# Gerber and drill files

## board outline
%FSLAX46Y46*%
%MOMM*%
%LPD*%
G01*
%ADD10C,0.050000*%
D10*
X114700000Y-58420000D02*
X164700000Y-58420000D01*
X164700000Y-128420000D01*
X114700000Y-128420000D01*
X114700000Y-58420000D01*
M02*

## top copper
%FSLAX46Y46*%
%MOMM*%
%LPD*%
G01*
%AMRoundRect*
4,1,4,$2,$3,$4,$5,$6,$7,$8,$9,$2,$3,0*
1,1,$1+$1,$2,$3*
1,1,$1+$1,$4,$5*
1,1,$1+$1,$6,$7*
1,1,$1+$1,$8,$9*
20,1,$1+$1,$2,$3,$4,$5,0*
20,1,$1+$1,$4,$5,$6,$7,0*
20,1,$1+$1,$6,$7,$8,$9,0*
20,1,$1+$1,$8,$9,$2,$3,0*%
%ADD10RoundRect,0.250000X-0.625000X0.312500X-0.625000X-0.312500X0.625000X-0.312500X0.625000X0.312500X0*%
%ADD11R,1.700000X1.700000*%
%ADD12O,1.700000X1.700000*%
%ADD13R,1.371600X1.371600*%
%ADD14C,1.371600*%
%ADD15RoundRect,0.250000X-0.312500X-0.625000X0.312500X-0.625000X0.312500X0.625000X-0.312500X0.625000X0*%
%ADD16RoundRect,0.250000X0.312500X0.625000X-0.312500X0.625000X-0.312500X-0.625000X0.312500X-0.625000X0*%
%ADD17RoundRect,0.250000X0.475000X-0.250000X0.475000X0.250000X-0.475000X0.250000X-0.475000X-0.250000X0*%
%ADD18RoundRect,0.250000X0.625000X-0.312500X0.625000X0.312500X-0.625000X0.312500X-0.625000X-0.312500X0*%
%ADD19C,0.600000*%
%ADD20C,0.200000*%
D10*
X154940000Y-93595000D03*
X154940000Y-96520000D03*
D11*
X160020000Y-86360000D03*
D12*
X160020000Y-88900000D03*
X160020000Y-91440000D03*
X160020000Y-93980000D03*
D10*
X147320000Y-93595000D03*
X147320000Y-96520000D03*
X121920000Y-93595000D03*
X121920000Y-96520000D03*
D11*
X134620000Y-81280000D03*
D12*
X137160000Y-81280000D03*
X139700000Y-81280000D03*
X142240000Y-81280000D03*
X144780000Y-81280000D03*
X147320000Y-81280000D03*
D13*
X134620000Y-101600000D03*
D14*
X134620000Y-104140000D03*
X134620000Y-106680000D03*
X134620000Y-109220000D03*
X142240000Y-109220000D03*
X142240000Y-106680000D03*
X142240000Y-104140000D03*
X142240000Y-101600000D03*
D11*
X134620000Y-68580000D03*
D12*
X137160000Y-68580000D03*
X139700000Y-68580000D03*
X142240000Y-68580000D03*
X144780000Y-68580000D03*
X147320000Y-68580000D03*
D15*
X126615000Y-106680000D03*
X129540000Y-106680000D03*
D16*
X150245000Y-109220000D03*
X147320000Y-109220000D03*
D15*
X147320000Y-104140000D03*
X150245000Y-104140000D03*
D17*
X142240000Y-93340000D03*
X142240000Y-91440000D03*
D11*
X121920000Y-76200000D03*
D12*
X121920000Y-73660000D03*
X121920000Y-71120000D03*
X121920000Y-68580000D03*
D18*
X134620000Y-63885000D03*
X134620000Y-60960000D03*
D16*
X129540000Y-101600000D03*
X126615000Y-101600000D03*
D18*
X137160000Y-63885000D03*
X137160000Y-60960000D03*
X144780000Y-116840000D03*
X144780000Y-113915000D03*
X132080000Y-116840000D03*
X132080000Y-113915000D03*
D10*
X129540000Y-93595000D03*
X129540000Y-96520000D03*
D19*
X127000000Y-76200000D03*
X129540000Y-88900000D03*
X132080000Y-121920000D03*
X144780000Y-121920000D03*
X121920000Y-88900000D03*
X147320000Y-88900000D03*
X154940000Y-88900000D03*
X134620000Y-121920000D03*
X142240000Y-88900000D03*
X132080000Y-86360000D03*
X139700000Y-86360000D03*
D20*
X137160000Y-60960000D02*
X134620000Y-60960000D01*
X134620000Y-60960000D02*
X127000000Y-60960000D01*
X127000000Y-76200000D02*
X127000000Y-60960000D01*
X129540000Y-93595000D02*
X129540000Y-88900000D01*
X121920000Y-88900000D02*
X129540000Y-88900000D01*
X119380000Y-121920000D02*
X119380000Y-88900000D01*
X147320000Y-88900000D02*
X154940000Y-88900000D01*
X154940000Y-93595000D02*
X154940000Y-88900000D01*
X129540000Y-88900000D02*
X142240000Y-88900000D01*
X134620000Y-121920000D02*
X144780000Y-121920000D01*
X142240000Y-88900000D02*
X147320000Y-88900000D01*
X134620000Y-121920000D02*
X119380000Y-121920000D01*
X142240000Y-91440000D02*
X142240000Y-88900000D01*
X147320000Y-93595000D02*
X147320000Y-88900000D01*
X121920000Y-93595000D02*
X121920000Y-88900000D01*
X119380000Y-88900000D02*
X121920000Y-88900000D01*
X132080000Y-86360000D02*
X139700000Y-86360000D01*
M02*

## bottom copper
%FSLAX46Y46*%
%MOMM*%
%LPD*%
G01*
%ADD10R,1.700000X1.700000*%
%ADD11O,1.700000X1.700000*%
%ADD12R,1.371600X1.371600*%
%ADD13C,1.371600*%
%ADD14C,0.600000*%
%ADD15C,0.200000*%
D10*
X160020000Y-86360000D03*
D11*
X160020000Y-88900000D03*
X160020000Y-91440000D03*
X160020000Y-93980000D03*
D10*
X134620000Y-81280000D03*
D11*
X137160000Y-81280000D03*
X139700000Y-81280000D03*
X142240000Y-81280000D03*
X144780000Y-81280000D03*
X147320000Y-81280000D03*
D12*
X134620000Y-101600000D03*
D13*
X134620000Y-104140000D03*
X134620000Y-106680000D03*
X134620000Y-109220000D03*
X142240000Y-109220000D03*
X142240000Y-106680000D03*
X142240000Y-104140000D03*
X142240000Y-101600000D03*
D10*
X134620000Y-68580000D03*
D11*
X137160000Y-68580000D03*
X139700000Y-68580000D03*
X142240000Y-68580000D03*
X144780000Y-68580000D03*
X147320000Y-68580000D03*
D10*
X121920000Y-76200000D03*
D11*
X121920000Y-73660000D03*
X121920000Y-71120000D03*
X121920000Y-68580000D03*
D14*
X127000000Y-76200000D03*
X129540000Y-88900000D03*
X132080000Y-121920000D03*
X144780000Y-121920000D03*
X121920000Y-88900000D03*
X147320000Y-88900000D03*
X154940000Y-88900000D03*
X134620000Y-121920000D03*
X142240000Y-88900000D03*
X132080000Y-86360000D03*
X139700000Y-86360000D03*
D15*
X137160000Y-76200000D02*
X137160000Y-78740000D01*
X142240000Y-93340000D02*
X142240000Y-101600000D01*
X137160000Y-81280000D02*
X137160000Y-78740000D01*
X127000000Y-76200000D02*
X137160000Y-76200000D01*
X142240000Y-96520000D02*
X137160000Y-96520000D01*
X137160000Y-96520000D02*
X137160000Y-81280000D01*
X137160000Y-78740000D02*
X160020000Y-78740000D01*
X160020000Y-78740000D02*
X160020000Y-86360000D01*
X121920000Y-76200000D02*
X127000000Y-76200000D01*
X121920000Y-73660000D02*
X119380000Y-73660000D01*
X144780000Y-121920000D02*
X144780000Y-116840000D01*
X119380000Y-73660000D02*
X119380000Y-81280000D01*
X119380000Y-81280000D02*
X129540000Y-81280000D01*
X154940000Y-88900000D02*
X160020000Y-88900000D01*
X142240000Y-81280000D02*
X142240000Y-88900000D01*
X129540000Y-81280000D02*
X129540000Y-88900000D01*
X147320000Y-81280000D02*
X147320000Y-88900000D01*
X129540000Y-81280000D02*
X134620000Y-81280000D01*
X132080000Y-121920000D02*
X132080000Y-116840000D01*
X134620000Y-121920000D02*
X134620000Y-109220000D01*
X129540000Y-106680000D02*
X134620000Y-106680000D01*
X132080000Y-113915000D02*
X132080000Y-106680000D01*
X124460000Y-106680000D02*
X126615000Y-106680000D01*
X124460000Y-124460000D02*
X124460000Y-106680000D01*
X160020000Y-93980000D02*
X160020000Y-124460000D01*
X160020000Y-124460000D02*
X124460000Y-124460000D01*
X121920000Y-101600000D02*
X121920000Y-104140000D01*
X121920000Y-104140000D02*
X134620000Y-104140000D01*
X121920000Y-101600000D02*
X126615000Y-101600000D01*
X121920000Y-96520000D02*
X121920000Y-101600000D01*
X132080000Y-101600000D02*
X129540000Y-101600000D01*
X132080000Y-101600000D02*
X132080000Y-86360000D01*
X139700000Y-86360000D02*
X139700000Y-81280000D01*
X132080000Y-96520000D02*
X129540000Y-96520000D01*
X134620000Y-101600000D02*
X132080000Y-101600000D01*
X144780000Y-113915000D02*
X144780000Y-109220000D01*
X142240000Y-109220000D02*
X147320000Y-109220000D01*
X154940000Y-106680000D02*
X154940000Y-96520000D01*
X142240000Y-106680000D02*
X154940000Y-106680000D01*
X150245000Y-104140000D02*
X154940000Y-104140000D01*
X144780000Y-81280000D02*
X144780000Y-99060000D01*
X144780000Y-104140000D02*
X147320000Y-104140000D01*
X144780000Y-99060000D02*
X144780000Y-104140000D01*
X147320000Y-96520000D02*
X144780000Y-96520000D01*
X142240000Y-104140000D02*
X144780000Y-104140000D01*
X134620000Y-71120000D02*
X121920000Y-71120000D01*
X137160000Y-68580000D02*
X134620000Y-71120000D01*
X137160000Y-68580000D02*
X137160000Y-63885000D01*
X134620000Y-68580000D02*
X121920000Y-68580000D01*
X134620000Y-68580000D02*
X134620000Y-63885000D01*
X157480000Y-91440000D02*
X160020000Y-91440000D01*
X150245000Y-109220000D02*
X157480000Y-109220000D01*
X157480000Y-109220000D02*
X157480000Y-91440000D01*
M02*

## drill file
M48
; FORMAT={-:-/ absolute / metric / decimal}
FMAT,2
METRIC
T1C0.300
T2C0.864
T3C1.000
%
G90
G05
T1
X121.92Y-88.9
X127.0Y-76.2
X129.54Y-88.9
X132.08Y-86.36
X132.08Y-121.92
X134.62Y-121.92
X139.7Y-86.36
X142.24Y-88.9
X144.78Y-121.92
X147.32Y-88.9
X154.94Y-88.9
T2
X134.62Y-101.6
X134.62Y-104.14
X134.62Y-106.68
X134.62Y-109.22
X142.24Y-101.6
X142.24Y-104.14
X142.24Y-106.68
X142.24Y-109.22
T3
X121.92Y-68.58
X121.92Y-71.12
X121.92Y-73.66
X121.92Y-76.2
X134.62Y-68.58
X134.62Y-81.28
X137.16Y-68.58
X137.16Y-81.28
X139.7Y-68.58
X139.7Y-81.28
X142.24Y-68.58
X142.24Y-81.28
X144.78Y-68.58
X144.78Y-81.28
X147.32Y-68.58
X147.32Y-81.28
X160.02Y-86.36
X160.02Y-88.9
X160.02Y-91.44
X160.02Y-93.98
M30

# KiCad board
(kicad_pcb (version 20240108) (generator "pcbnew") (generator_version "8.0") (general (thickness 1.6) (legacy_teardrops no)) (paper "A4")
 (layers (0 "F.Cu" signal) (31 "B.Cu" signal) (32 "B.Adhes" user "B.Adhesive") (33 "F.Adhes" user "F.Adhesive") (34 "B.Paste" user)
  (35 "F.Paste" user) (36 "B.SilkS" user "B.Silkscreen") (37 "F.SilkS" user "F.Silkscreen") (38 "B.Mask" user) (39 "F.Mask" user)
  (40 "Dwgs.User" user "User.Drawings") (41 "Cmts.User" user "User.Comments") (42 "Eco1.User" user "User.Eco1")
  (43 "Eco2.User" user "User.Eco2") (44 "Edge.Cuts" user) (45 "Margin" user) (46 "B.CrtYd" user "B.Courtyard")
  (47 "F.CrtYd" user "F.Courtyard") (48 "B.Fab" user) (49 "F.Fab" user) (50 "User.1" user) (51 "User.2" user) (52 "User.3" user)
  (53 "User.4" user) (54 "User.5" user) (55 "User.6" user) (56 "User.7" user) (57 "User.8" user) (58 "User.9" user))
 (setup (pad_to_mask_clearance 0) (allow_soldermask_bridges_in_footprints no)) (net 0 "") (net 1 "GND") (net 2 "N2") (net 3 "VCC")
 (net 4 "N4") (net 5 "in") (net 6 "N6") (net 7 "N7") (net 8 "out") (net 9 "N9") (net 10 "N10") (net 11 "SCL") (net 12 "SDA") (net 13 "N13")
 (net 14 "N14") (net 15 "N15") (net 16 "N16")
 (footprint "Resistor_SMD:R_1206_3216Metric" (layer "F.Cu") (at 154.94 95.0575 -90)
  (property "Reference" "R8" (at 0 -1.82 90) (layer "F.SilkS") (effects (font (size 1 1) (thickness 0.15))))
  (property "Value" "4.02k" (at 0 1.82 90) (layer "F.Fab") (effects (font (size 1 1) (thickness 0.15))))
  (pad "1" smd roundrect (at -1.4625 0 270) (size 1.125 1.75) (layers "F.Cu" "F.Paste" "F.Mask") (roundrect_rratio 0.222222) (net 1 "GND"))
  (pad "2" smd roundrect (at 1.4625 0 270) (size 1.125 1.75) (layers "F.Cu" "F.Paste" "F.Mask") (roundrect_rratio 0.222222) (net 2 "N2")))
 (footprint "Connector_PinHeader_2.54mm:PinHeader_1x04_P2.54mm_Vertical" (layer "F.Cu") (at 160.02 86.36)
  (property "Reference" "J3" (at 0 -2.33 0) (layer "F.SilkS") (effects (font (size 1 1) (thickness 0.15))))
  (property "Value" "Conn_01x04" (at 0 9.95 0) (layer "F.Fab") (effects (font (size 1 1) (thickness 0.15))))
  (pad "1" thru_hole rect (at 0 0) (size 1.7 1.7) (drill 1) (layers "*.Cu" "*.Mask") (remove_unused_layers no) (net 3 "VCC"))
  (pad "2" thru_hole oval (at 0 2.54) (size 1.7 1.7) (drill 1) (layers "*.Cu" "*.Mask") (remove_unused_layers no) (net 1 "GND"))
  (pad "3" thru_hole oval (at 0 5.08) (size 1.7 1.7) (drill 1) (layers "*.Cu" "*.Mask") (remove_unused_layers no) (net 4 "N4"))
  (pad "4" thru_hole oval (at 0 7.62) (size 1.7 1.7) (drill 1) (layers "*.Cu" "*.Mask") (remove_unused_layers no) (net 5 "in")))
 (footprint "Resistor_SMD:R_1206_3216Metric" (layer "F.Cu") (at 147.32 95.0575 -90)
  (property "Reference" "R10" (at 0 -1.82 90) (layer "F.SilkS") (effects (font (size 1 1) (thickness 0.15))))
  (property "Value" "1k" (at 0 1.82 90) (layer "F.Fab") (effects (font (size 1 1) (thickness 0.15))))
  (pad "1" smd roundrect (at -1.4625 0 270) (size 1.125 1.75) (layers "F.Cu" "F.Paste" "F.Mask") (roundrect_rratio 0.222222) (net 1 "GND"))
  (pad "2" smd roundrect (at 1.4625 0 270) (size 1.125 1.75) (layers "F.Cu" "F.Paste" "F.Mask") (roundrect_rratio 0.222222) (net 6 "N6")))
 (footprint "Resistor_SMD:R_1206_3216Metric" (layer "F.Cu") (at 121.92 95.0575 -90)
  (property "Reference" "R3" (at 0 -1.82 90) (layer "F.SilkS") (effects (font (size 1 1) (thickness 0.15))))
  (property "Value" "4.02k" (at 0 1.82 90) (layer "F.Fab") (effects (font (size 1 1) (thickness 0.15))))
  (pad "1" smd roundrect (at -1.4625 0 270) (size 1.125 1.75) (layers "F.Cu" "F.Paste" "F.Mask") (roundrect_rratio 0.222222) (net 1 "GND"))
  (pad "2" smd roundrect (at 1.4625 0 270) (size 1.125 1.75) (layers "F.Cu" "F.Paste" "F.Mask") (roundrect_rratio 0.222222) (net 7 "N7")))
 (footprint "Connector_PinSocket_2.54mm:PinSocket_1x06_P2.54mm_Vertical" (layer "F.Cu") (at 134.62 81.28 90)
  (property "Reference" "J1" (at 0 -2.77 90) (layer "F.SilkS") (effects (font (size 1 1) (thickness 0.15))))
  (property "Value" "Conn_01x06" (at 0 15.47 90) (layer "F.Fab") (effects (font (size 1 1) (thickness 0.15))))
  (pad "1" thru_hole rect (at 0 0 90) (size 1.7 1.7) (drill 1) (layers "*.Cu" "*.Mask") (remove_unused_layers no) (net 1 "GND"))
  (pad "2" thru_hole oval (at 0 2.54 90) (size 1.7 1.7) (drill 1) (layers "*.Cu" "*.Mask") (remove_unused_layers no) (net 3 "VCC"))
  (pad "3" thru_hole oval (at 0 5.08 90) (size 1.7 1.7) (drill 1) (layers "*.Cu" "*.Mask") (remove_unused_layers no) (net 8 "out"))
  (pad "4" thru_hole oval (at 0 7.62 90) (size 1.7 1.7) (drill 1) (layers "*.Cu" "*.Mask") (remove_unused_layers no) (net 1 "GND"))
  (pad "5" thru_hole oval (at 0 10.16 90) (size 1.7 1.7) (drill 1) (layers "*.Cu" "*.Mask") (remove_unused_layers no) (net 6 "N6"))
  (pad "6" thru_hole oval (at 0 12.7 90) (size 1.7 1.7) (drill 1) (layers "*.Cu" "*.Mask") (remove_unused_layers no) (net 1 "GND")))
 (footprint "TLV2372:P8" (layer "F.Cu") (at 142.24 109.22)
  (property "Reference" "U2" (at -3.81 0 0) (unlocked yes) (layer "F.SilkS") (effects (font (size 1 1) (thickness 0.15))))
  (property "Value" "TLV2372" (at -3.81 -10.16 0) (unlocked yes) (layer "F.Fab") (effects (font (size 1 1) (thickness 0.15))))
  (pad "1" thru_hole rect (at -7.62 -7.62) (size 1.3716 1.3716) (drill 0.8636) (layers "*.Cu" "*.Mask") (remove_unused_layers no)
   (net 8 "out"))
  (pad "2" thru_hole circle (at -7.62 -5.08) (size 1.3716 1.3716) (drill 0.8636) (layers "*.Cu" "*.Mask") (remove_unused_layers no)
   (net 7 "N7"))
  (pad "3" thru_hole circle (at -7.62 -2.54) (size 1.3716 1.3716) (drill 0.8636) (layers "*.Cu" "*.Mask") (remove_unused_layers no)
   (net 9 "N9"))
  (pad "4" thru_hole circle (at -7.62 0) (size 1.3716 1.3716) (drill 0.8636) (layers "*.Cu" "*.Mask") (remove_unused_layers no)
   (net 1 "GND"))
  (pad "5" thru_hole circle (at 0 0) (size 1.3716 1.3716) (drill 0.8636) (layers "*.Cu" "*.Mask") (remove_unused_layers no) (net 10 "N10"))
  (pad "6" thru_hole circle (at 0 -2.54) (size 1.3716 1.3716) (drill 0.8636) (layers "*.Cu" "*.Mask") (remove_unused_layers no) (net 2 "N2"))
  (pad "7" thru_hole circle (at 0 -5.08) (size 1.3716 1.3716) (drill 0.8636) (layers "*.Cu" "*.Mask") (remove_unused_layers no) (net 6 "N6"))
  (pad "8" thru_hole circle (at 0 -7.62) (size 1.3716 1.3716) (drill 0.8636) (layers "*.Cu" "*.Mask") (remove_unused_layers no)
   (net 3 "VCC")))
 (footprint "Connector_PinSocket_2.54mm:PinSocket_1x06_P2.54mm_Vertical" (layer "F.Cu") (at 134.62 68.58 90)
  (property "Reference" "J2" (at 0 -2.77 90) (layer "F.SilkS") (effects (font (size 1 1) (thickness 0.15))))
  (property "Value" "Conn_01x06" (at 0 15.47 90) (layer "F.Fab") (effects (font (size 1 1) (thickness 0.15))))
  (pad "1" thru_hole rect (at 0 0 90) (size 1.7 1.7) (drill 1) (layers "*.Cu" "*.Mask") (remove_unused_layers no) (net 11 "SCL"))
  (pad "2" thru_hole oval (at 0 2.54 90) (size 1.7 1.7) (drill 1) (layers "*.Cu" "*.Mask") (remove_unused_layers no) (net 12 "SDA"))
  (pad "3" thru_hole oval (at 0 5.08 90) (size 1.7 1.7) (drill 1) (layers "*.Cu" "*.Mask") (remove_unused_layers no) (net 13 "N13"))
  (pad "4" thru_hole oval (at 0 7.62 90) (size 1.7 1.7) (drill 1) (layers "*.Cu" "*.Mask") (remove_unused_layers no) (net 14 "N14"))
  (pad "5" thru_hole oval (at 0 10.16 90) (size 1.7 1.7) (drill 1) (layers "*.Cu" "*.Mask") (remove_unused_layers no) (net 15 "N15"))
  (pad "6" thru_hole oval (at 0 12.7 90) (size 1.7 1.7) (drill 1) (layers "*.Cu" "*.Mask") (remove_unused_layers no) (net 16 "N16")))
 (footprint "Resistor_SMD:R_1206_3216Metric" (layer "F.Cu") (at 128.0775 106.68)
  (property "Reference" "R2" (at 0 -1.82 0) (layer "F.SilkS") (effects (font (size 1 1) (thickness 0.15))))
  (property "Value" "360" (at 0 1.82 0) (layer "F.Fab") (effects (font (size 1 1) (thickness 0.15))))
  (pad "1" smd roundrect (at -1.4625 0) (size 1.125 1.75) (layers "F.Cu" "F.Paste" "F.Mask") (roundrect_rratio 0.222222) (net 5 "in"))
  (pad "2" smd roundrect (at 1.4625 0) (size 1.125 1.75) (layers "F.Cu" "F.Paste" "F.Mask") (roundrect_rratio 0.222222) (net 9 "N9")))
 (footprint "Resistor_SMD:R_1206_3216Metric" (layer "F.Cu") (at 148.7825 109.22 180)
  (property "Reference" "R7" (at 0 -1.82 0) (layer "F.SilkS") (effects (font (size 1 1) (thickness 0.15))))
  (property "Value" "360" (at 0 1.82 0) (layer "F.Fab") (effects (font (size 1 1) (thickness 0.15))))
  (pad "1" smd roundrect (at -1.4625 0 180) (size 1.125 1.75) (layers "F.Cu" "F.Paste" "F.Mask") (roundrect_rratio 0.222222) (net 4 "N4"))
  (pad "2" smd roundrect (at 1.4625 0 180) (size 1.125 1.75) (layers "F.Cu" "F.Paste" "F.Mask") (roundrect_rratio 0.222222) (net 10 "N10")))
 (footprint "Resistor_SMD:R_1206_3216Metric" (layer "F.Cu") (at 148.7825 104.14)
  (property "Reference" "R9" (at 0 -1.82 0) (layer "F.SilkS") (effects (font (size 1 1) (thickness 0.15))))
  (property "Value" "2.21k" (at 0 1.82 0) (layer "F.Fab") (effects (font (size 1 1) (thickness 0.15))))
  (pad "1" smd roundrect (at -1.4625 0) (size 1.125 1.75) (layers "F.Cu" "F.Paste" "F.Mask") (roundrect_rratio 0.222222) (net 6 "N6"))
  (pad "2" smd roundrect (at 1.4625 0) (size 1.125 1.75) (layers "F.Cu" "F.Paste" "F.Mask") (roundrect_rratio 0.222222) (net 2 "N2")))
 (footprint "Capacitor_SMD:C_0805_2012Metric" (layer "F.Cu") (at 142.24 92.39 90)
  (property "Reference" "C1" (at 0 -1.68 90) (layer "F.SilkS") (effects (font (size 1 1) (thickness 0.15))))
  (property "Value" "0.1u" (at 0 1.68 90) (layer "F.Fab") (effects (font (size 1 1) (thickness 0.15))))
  (pad "1" smd roundrect (at -0.95 0 90) (size 1 1.45) (layers "F.Cu" "F.Paste" "F.Mask") (roundrect_rratio 0.25) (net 3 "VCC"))
  (pad "2" smd roundrect (at 0.95 0 90) (size 1 1.45) (layers "F.Cu" "F.Paste" "F.Mask") (roundrect_rratio 0.25) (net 1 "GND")))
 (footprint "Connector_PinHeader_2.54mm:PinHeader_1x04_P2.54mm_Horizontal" (layer "F.Cu") (at 121.92 76.2 180)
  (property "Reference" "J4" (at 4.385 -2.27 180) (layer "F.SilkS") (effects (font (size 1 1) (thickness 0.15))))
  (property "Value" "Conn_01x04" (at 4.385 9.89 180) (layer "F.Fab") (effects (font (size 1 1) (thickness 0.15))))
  (pad "1" thru_hole rect (at 0 0 180) (size 1.7 1.7) (drill 1) (layers "*.Cu" "*.Mask") (remove_unused_layers no) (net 3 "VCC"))
  (pad "2" thru_hole oval (at 0 2.54 180) (size 1.7 1.7) (drill 1) (layers "*.Cu" "*.Mask") (remove_unused_layers no) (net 1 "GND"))
  (pad "3" thru_hole oval (at 0 5.08 180) (size 1.7 1.7) (drill 1) (layers "*.Cu" "*.Mask") (remove_unused_layers no) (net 12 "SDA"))
  (pad "4" thru_hole oval (at 0 7.62 180) (size 1.7 1.7) (drill 1) (layers "*.Cu" "*.Mask") (remove_unused_layers no) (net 11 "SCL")))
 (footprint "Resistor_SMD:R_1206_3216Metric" (layer "F.Cu") (at 134.62 62.4225 90)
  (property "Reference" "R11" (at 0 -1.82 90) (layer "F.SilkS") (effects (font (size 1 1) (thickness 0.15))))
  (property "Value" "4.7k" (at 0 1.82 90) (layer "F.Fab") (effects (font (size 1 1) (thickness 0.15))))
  (pad "1" smd roundrect (at -1.4625 0 90) (size 1.125 1.75) (layers "F.Cu" "F.Paste" "F.Mask") (roundrect_rratio 0.222222) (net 11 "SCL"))
  (pad "2" smd roundrect (at 1.4625 0 90) (size 1.125 1.75) (layers "F.Cu" "F.Paste" "F.Mask") (roundrect_rratio 0.222222) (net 3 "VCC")))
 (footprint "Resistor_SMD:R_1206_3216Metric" (layer "F.Cu") (at 128.0775 101.6 180)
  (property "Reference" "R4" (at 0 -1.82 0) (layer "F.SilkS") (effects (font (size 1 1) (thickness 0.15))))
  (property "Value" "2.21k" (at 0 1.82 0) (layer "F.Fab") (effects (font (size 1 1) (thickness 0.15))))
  (pad "1" smd roundrect (at -1.4625 0 180) (size 1.125 1.75) (layers "F.Cu" "F.Paste" "F.Mask") (roundrect_rratio 0.222222) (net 8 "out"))
  (pad "2" smd roundrect (at 1.4625 0 180) (size 1.125 1.75) (layers "F.Cu" "F.Paste" "F.Mask") (roundrect_rratio 0.222222) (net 7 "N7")))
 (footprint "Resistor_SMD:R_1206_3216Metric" (layer "F.Cu") (at 137.16 62.4225 90)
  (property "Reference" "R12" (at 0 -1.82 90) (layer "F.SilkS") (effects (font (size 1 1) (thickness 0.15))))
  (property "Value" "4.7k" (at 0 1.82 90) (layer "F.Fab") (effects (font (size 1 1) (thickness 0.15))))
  (pad "1" smd roundrect (at -1.4625 0 90) (size 1.125 1.75) (layers "F.Cu" "F.Paste" "F.Mask") (roundrect_rratio 0.222222) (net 12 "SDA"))
  (pad "2" smd roundrect (at 1.4625 0 90) (size 1.125 1.75) (layers "F.Cu" "F.Paste" "F.Mask") (roundrect_rratio 0.222222) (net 3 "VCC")))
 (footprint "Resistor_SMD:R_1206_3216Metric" (layer "F.Cu") (at 144.78 115.3775 90)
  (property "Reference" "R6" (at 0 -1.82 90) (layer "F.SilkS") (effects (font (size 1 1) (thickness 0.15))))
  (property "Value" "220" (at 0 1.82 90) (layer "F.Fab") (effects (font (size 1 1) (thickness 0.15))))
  (pad "1" smd roundrect (at -1.4625 0 90) (size 1.125 1.75) (layers "F.Cu" "F.Paste" "F.Mask") (roundrect_rratio 0.222222) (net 1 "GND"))
  (pad "2" smd roundrect (at 1.4625 0 90) (size 1.125 1.75) (layers "F.Cu" "F.Paste" "F.Mask") (roundrect_rratio 0.222222) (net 10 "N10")))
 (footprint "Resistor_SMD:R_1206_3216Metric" (layer "F.Cu") (at 132.08 115.3775 90)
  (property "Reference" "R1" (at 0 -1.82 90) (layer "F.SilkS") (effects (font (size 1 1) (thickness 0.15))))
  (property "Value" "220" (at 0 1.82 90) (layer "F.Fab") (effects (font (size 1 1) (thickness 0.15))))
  (pad "1" smd roundrect (at -1.4625 0 90) (size 1.125 1.75) (layers "F.Cu" "F.Paste" "F.Mask") (roundrect_rratio 0.222222) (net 1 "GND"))
  (pad "2" smd roundrect (at 1.4625 0 90) (size 1.125 1.75) (layers "F.Cu" "F.Paste" "F.Mask") (roundrect_rratio 0.222222) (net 9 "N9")))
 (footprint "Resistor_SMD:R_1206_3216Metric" (layer "F.Cu") (at 129.54 95.0575 -90)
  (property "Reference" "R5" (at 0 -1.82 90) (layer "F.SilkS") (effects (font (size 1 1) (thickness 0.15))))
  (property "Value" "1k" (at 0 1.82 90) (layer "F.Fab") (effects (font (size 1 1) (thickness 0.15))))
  (pad "1" smd roundrect (at -1.4625 0 270) (size 1.125 1.75) (layers "F.Cu" "F.Paste" "F.Mask") (roundrect_rratio 0.222222) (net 1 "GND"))
  (pad "2" smd roundrect (at 1.4625 0 270) (size 1.125 1.75) (layers "F.Cu" "F.Paste" "F.Mask") (roundrect_rratio 0.222222) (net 8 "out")))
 (gr_rect (start 114.7 58.42) (end 164.7 128.42) (stroke (width 0.05) (type default)) (fill none) (layer "Edge.Cuts"))
 (segment (start 137.16 60.96) (end 134.62 60.96) (width 0.2) (layer "F.Cu") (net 3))
 (segment (start 134.62 60.96) (end 127 60.96) (width 0.2) (layer "F.Cu") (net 3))
 (segment (start 127 76.2) (end 127 60.96) (width 0.2) (layer "F.Cu") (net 3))
 (via (at 127 76.2) (size 0.6) (drill 0.3) (layers "F.Cu" "B.Cu") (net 3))
 (segment (start 137.16 76.2) (end 137.16 78.74) (width 0.2) (layer "B.Cu") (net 3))
 (segment (start 142.24 93.34) (end 142.24 101.6) (width 0.2) (layer "B.Cu") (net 3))
 (segment (start 137.16 81.28) (end 137.16 78.74) (width 0.2) (layer "B.Cu") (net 3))
 (segment (start 127 76.2) (end 137.16 76.2) (width 0.2) (layer "B.Cu") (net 3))
 (segment (start 142.24 96.52) (end 137.16 96.52) (width 0.2) (layer "B.Cu") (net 3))
 (segment (start 137.16 96.52) (end 137.16 81.28) (width 0.2) (layer "B.Cu") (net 3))
 (segment (start 137.16 78.74) (end 160.02 78.74) (width 0.2) (layer "B.Cu") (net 3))
 (segment (start 160.02 78.74) (end 160.02 86.36) (width 0.2) (layer "B.Cu") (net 3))
 (segment (start 121.92 76.2) (end 127 76.2) (width 0.2) (layer "B.Cu") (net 3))
 (segment (start 129.54 93.595) (end 129.54 88.9) (width 0.2) (layer "F.Cu") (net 1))
 (segment (start 121.92 88.9) (end 129.54 88.9) (width 0.2) (layer "F.Cu") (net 1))
 (segment (start 119.38 121.92) (end 119.38 88.9) (width 0.2) (layer "F.Cu") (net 1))
 (segment (start 147.32 88.9) (end 154.94 88.9) (width 0.2) (layer "F.Cu") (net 1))
 (segment (start 154.94 93.595) (end 154.94 88.9) (width 0.2) (layer "F.Cu") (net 1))
 (segment (start 129.54 88.9) (end 142.24 88.9) (width 0.2) (layer "F.Cu") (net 1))
 (segment (start 134.62 121.92) (end 144.78 121.92) (width 0.2) (layer "F.Cu") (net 1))
 (segment (start 142.24 88.9) (end 147.32 88.9) (width 0.2) (layer "F.Cu") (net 1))
 (segment (start 134.62 121.92) (end 119.38 121.92) (width 0.2) (layer "F.Cu") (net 1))
 (segment (start 142.24 91.44) (end 142.24 88.9) (width 0.2) (layer "F.Cu") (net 1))
 (segment (start 147.32 93.595) (end 147.32 88.9) (width 0.2) (layer "F.Cu") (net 1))
 (segment (start 121.92 93.595) (end 121.92 88.9) (width 0.2) (layer "F.Cu") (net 1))
 (segment (start 119.38 88.9) (end 121.92 88.9) (width 0.2) (layer "F.Cu") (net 1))
 (via (at 129.54 88.9) (size 0.6) (drill 0.3) (layers "F.Cu" "B.Cu") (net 1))
 (via (at 132.08 121.92) (size 0.6) (drill 0.3) (layers "F.Cu" "B.Cu") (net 1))
 (via (at 144.78 121.92) (size 0.6) (drill 0.3) (layers "F.Cu" "B.Cu") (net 1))
 (via (at 121.92 88.9) (size 0.6) (drill 0.3) (layers "F.Cu" "B.Cu") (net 1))
 (via (at 147.32 88.9) (size 0.6) (drill 0.3) (layers "F.Cu" "B.Cu") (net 1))
 (via (at 154.94 88.9) (size 0.6) (drill 0.3) (layers "F.Cu" "B.Cu") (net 1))
 (via (at 134.62 121.92) (size 0.6) (drill 0.3) (layers "F.Cu" "B.Cu") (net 1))
 (via (at 142.24 88.9) (size 0.6) (drill 0.3) (layers "F.Cu" "B.Cu") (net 1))
 (segment (start 121.92 73.66) (end 119.38 73.66) (width 0.2) (layer "B.Cu") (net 1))
 (segment (start 144.78 121.92) (end 144.78 116.84) (width 0.2) (layer "B.Cu") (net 1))
 (segment (start 119.38 73.66) (end 119.38 81.28) (width 0.2) (layer "B.Cu") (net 1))
 (segment (start 119.38 81.28) (end 129.54 81.28) (width 0.2) (layer "B.Cu") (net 1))
 (segment (start 154.94 88.9) (end 160.02 88.9) (width 0.2) (layer "B.Cu") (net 1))
 (segment (start 142.24 81.28) (end 142.24 88.9) (width 0.2) (layer "B.Cu") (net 1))
 (segment (start 129.54 81.28) (end 129.54 88.9) (width 0.2) (layer "B.Cu") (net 1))
 (segment (start 147.32 81.28) (end 147.32 88.9) (width 0.2) (layer "B.Cu") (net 1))
 (segment (start 129.54 81.28) (end 134.62 81.28) (width 0.2) (layer "B.Cu") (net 1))
 (segment (start 132.08 121.92) (end 132.08 116.84) (width 0.2) (layer "B.Cu") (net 1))
 (segment (start 134.62 121.92) (end 134.62 109.22) (width 0.2) (layer "B.Cu") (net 1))
 (segment (start 129.54 106.68) (end 134.62 106.68) (width 0.2) (layer "B.Cu") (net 9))
 (segment (start 132.08 113.915) (end 132.08 106.68) (width 0.2) (layer "B.Cu") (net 9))
 (segment (start 124.46 106.68) (end 126.615 106.68) (width 0.2) (layer "B.Cu") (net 5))
 (segment (start 124.46 124.46) (end 124.46 106.68) (width 0.2) (layer "B.Cu") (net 5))
 (segment (start 160.02 93.98) (end 160.02 124.46) (width 0.2) (layer "B.Cu") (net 5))
 (segment (start 160.02 124.46) (end 124.46 124.46) (width 0.2) (layer "B.Cu") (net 5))
 (segment (start 121.92 101.6) (end 121.92 104.14) (width 0.2) (layer "B.Cu") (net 7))
 (segment (start 121.92 104.14) (end 134.62 104.14) (width 0.2) (layer "B.Cu") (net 7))
 (segment (start 121.92 101.6) (end 126.615 101.6) (width 0.2) (layer "B.Cu") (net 7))
 (segment (start 121.92 96.52) (end 121.92 101.6) (width 0.2) (layer "B.Cu") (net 7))
 (segment (start 132.08 86.36) (end 139.7 86.36) (width 0.2) (layer "F.Cu") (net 8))
 (via (at 132.08 86.36) (size 0.6) (drill 0.3) (layers "F.Cu" "B.Cu") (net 8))
 (via (at 139.7 86.36) (size 0.6) (drill 0.3) (layers "F.Cu" "B.Cu") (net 8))
 (segment (start 132.08 101.6) (end 129.54 101.6) (width 0.2) (layer "B.Cu") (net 8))
 (segment (start 132.08 101.6) (end 132.08 86.36) (width 0.2) (layer "B.Cu") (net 8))
 (segment (start 139.7 86.36) (end 139.7 81.28) (width 0.2) (layer "B.Cu") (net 8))
 (segment (start 132.08 96.52) (end 129.54 96.52) (width 0.2) (layer "B.Cu") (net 8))
 (segment (start 134.62 101.6) (end 132.08 101.6) (width 0.2) (layer "B.Cu") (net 8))
 (segment (start 144.78 113.915) (end 144.78 109.22) (width 0.2) (layer "B.Cu") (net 10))
 (segment (start 142.24 109.22) (end 147.32 109.22) (width 0.2) (layer "B.Cu") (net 10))
 (segment (start 154.94 106.68) (end 154.94 96.52) (width 0.2) (layer "B.Cu") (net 2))
 (segment (start 142.24 106.68) (end 154.94 106.68) (width 0.2) (layer "B.Cu") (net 2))
 (segment (start 150.245 104.14) (end 154.94 104.14) (width 0.2) (layer "B.Cu") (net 2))
 (segment (start 144.78 81.28) (end 144.78 99.06) (width 0.2) (layer "B.Cu") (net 6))
 (segment (start 144.78 104.14) (end 147.32 104.14) (width 0.2) (layer "B.Cu") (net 6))
 (segment (start 144.78 99.06) (end 144.78 104.14) (width 0.2) (layer "B.Cu") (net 6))
 (segment (start 147.32 96.52) (end 144.78 96.52) (width 0.2) (layer "B.Cu") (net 6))
 (segment (start 142.24 104.14) (end 144.78 104.14) (width 0.2) (layer "B.Cu") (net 6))
 (segment (start 134.62 71.12) (end 121.92 71.12) (width 0.2) (layer "B.Cu") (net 12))
 (segment (start 137.16 68.58) (end 134.62 71.12) (width 0.2) (layer "B.Cu") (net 12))
 (segment (start 137.16 68.58) (end 137.16 63.885) (width 0.2) (layer "B.Cu") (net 12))
 (segment (start 134.62 68.58) (end 121.92 68.58) (width 0.2) (layer "B.Cu") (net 11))
 (segment (start 134.62 68.58) (end 134.62 63.885) (width 0.2) (layer "B.Cu") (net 11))
 (segment (start 157.48 91.44) (end 160.02 91.44) (width 0.2) (layer "B.Cu") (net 4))
 (segment (start 150.245 109.22) (end 157.48 109.22) (width 0.2) (layer "B.Cu") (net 4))
 (segment (start 157.48 109.22) (end 157.48 91.44) (width 0.2) (layer "B.Cu") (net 4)))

